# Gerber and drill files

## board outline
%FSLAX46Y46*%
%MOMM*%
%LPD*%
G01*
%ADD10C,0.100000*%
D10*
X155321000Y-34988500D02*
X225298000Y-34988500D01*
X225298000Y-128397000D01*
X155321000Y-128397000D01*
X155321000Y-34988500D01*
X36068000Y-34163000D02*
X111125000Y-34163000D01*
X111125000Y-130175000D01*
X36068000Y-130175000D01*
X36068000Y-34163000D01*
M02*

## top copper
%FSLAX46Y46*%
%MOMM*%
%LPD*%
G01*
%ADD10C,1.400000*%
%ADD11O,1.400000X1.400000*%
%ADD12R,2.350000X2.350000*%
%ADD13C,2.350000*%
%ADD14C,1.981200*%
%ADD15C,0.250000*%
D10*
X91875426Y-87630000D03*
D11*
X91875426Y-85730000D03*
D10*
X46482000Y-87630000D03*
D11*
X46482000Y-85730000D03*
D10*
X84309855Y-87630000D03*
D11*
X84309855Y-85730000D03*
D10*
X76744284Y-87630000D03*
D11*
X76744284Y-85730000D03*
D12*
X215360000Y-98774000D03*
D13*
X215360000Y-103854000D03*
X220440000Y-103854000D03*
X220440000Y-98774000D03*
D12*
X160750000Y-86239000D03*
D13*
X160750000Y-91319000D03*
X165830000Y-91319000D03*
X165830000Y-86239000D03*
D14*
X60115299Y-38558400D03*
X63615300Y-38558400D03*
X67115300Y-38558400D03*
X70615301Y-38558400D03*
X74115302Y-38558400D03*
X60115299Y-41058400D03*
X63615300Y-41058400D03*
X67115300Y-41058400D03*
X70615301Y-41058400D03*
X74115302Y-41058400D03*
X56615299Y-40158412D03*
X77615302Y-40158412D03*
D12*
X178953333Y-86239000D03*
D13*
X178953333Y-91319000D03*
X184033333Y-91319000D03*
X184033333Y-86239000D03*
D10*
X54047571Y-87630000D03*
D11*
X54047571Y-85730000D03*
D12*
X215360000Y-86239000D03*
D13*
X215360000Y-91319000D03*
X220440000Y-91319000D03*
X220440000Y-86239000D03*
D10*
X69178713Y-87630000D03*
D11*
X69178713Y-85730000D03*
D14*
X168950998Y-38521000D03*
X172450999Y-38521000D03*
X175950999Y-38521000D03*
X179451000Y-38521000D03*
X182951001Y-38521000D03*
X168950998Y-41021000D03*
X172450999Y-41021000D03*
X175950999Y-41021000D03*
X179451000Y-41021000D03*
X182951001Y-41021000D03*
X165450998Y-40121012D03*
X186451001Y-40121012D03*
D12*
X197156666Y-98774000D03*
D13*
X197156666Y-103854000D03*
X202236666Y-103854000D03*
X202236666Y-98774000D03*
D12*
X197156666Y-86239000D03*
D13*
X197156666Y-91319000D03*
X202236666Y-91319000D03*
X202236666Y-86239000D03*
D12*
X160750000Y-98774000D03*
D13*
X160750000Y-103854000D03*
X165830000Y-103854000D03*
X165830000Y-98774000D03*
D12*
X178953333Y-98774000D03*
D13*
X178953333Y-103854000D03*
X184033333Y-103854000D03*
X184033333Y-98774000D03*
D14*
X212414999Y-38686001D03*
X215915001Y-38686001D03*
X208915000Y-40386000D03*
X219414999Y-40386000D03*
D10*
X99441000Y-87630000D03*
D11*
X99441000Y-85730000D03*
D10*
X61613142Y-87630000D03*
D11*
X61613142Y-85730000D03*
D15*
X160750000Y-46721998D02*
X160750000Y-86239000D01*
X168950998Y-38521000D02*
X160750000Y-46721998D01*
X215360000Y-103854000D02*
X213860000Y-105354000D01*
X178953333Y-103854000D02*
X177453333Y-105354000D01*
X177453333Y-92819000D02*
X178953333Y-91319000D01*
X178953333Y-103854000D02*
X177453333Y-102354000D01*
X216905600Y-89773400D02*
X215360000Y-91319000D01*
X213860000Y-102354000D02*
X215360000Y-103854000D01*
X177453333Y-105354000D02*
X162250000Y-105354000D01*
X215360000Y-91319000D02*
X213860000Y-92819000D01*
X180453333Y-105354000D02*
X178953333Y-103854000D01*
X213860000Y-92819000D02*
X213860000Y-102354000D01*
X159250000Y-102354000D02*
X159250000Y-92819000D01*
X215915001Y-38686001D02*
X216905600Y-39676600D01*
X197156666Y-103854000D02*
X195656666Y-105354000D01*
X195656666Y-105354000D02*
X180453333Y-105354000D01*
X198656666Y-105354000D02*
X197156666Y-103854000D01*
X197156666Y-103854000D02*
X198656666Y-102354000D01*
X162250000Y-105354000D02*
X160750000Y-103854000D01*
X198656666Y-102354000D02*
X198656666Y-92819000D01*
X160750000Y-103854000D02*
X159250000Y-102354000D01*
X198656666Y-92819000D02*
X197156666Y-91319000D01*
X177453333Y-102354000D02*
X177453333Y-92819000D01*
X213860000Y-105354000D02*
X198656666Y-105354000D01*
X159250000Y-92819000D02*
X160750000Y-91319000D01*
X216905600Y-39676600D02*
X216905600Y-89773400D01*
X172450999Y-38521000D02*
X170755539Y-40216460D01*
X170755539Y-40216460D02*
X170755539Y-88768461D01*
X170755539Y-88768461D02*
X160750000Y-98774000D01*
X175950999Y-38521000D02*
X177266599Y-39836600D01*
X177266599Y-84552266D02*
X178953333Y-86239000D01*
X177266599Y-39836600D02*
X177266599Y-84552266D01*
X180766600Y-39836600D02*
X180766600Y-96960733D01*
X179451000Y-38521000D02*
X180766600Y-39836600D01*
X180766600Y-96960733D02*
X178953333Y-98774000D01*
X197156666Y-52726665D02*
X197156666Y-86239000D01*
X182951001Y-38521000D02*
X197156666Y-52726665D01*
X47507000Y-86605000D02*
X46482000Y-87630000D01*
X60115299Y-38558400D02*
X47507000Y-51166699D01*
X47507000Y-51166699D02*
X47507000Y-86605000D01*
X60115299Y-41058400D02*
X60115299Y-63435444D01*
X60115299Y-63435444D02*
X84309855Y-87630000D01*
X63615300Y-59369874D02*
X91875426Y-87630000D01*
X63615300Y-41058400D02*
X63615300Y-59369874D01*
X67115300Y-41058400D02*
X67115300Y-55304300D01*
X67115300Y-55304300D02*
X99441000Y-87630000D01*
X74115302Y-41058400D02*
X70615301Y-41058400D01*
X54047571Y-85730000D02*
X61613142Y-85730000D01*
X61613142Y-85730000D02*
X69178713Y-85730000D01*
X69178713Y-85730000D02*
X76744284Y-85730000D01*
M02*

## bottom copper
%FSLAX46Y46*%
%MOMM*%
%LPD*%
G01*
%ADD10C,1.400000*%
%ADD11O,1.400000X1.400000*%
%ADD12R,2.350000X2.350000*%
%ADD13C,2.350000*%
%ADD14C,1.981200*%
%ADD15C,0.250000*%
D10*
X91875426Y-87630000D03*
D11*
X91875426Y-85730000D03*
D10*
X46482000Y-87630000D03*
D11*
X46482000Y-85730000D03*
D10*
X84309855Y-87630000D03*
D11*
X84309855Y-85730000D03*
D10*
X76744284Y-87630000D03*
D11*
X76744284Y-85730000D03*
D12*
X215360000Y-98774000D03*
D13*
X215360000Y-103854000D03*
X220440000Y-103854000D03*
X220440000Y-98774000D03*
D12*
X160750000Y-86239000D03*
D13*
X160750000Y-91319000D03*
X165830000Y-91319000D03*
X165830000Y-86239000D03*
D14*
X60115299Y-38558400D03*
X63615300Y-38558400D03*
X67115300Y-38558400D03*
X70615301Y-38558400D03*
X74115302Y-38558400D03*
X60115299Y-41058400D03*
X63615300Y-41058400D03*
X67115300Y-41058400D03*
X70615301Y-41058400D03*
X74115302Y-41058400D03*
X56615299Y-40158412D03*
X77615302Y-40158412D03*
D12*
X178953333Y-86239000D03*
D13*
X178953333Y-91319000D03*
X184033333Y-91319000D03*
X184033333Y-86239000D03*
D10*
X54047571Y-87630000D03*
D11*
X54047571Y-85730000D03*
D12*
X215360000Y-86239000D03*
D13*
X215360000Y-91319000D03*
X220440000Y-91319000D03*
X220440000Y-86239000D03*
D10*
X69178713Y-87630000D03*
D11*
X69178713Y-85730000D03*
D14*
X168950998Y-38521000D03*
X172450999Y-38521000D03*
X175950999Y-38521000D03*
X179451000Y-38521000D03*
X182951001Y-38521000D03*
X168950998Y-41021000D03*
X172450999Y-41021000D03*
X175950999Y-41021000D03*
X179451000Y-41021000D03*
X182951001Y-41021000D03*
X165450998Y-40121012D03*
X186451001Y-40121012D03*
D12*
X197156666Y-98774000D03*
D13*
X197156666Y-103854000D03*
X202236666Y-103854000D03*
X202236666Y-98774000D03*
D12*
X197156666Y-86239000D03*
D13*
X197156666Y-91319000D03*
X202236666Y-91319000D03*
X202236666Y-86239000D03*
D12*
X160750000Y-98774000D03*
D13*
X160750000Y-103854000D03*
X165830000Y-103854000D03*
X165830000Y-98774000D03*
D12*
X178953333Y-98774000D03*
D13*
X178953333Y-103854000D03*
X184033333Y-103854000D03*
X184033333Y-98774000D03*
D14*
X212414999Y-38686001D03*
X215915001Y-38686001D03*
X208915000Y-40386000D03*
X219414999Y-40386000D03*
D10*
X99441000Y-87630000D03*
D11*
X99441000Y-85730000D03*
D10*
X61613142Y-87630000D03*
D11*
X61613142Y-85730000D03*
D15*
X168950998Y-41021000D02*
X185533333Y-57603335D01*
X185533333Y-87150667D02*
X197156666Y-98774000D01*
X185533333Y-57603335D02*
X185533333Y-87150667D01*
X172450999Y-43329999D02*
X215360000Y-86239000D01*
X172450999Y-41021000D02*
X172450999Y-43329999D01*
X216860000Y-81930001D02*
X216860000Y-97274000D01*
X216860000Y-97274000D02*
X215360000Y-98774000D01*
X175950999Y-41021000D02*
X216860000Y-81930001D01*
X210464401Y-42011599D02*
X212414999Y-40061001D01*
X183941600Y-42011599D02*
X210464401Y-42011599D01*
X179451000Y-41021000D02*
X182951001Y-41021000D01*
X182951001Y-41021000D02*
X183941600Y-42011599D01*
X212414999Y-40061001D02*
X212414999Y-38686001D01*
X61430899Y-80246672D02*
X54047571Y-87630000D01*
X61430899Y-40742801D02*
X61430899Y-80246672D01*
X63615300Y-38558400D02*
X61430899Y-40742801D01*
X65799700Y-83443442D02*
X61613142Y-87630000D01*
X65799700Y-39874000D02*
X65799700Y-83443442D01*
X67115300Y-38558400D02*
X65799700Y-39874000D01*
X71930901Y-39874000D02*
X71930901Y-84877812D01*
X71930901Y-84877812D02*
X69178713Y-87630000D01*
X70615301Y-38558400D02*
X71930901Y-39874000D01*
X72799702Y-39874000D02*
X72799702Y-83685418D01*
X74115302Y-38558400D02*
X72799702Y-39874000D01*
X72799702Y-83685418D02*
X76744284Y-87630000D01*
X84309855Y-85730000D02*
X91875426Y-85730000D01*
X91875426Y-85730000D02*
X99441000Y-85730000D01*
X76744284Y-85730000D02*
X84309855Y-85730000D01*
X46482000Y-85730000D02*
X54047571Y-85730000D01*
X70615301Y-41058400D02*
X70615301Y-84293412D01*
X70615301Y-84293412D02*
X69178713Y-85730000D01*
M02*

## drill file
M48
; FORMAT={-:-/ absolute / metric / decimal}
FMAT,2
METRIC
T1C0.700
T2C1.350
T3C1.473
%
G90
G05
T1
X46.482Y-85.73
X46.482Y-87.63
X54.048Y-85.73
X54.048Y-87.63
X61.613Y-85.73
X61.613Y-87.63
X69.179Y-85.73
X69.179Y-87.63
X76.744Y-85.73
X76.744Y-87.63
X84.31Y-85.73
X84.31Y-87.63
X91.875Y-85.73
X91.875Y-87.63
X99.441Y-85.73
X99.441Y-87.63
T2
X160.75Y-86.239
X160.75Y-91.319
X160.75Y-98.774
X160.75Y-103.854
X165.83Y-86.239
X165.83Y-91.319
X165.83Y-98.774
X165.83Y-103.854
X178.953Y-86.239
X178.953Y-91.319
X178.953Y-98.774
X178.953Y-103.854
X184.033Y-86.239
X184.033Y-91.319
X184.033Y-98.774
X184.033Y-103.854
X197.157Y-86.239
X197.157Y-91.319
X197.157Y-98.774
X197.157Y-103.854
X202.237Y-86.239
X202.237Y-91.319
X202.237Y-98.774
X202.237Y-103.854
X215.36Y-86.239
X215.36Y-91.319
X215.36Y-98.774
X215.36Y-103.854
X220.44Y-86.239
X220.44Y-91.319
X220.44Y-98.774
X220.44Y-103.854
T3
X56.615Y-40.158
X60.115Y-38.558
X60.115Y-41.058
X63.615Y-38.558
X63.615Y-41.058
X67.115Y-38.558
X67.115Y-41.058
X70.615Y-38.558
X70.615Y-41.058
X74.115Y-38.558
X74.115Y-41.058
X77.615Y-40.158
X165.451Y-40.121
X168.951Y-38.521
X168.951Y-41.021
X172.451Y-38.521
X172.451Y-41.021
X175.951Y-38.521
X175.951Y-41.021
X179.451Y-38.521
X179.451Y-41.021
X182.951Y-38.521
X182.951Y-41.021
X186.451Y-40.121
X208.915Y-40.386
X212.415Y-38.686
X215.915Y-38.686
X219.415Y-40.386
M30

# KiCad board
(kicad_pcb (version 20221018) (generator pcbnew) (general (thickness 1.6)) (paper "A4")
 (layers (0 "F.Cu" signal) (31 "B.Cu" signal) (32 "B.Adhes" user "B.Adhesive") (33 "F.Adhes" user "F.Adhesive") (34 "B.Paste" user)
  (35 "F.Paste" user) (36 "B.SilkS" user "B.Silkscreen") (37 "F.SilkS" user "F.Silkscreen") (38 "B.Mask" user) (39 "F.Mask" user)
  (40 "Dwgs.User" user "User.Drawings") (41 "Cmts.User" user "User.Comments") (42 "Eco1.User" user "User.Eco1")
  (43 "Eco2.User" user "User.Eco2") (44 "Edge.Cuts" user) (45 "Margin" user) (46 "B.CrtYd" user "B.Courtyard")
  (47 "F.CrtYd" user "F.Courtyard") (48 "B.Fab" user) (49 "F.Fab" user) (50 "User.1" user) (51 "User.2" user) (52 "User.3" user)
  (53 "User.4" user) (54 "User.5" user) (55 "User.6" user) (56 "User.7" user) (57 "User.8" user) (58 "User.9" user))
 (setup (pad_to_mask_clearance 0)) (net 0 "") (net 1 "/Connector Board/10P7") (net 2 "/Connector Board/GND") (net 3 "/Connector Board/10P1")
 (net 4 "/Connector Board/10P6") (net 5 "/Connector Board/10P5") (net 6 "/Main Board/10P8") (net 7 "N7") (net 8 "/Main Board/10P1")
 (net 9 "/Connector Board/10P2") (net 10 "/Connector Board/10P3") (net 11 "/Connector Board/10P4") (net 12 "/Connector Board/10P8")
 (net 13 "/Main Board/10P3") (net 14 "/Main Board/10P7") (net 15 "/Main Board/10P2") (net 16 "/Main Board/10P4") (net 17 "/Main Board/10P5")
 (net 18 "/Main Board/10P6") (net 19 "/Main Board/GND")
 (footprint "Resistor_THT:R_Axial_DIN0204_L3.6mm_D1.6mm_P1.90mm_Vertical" (layer "F.Cu") (at 91.875426 87.63 90)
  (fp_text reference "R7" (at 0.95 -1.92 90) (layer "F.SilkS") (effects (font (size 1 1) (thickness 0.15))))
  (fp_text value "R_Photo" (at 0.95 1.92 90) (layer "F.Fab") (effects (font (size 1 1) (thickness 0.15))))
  (pad "1" thru_hole circle (at 0 0 90) (size 1.4 1.4) (drill 0.7) (layers "*.Cu" "*.Mask") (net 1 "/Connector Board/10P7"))
  (pad "2" thru_hole oval (at 1.9 0 90) (size 1.4 1.4) (drill 0.7) (layers "*.Cu" "*.Mask") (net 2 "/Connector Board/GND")))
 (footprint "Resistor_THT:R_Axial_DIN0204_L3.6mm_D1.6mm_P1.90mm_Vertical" (layer "F.Cu") (at 46.482 87.63 90)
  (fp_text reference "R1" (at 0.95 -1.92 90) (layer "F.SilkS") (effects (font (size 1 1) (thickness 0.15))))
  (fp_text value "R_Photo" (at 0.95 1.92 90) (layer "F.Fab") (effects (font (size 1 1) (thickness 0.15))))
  (pad "1" thru_hole circle (at 0 0 90) (size 1.4 1.4) (drill 0.7) (layers "*.Cu" "*.Mask") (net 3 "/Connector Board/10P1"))
  (pad "2" thru_hole oval (at 1.9 0 90) (size 1.4 1.4) (drill 0.7) (layers "*.Cu" "*.Mask") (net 2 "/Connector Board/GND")))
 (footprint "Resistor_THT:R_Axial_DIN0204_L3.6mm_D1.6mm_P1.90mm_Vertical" (layer "F.Cu") (at 84.309855 87.63 90)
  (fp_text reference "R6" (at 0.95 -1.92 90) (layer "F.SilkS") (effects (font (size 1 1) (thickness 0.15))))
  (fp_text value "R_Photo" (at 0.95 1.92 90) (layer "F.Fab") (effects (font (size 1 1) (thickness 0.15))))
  (pad "1" thru_hole circle (at 0 0 90) (size 1.4 1.4) (drill 0.7) (layers "*.Cu" "*.Mask") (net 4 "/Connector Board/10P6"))
  (pad "2" thru_hole oval (at 1.9 0 90) (size 1.4 1.4) (drill 0.7) (layers "*.Cu" "*.Mask") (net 2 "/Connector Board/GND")))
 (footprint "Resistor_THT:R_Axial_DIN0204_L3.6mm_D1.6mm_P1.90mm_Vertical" (layer "F.Cu") (at 76.744284 87.63 90)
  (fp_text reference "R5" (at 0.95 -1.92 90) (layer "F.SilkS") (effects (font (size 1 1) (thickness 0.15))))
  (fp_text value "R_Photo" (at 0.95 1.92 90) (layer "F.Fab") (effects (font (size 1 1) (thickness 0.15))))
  (pad "1" thru_hole circle (at 0 0 90) (size 1.4 1.4) (drill 0.7) (layers "*.Cu" "*.Mask") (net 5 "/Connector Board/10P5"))
  (pad "2" thru_hole oval (at 1.9 0 90) (size 1.4 1.4) (drill 0.7) (layers "*.Cu" "*.Mask") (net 2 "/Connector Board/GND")))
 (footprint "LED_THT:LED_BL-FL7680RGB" (layer "F.Cu") (at 215.36 98.774)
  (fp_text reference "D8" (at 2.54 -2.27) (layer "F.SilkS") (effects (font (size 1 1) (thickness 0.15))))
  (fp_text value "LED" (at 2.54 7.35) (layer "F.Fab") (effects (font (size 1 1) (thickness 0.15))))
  (pad "1" thru_hole rect (at 0 0) (size 2.35 2.35) (drill 1.35) (layers "*.Cu" "*.Mask") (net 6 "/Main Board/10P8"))
  (pad "2" thru_hole circle (at 0 5.08) (size 2.35 2.35) (drill 1.35) (layers "*.Cu" "*.Mask") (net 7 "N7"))
  (pad "3" thru_hole circle (at 5.08 5.08) (size 2.35 2.35) (drill 1.35) (layers "*.Cu" "*.Mask"))
  (pad "4" thru_hole circle (at 5.08 0) (size 2.35 2.35) (drill 1.35) (layers "*.Cu" "*.Mask")))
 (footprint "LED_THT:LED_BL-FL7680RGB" (layer "F.Cu") (at 160.75 86.239)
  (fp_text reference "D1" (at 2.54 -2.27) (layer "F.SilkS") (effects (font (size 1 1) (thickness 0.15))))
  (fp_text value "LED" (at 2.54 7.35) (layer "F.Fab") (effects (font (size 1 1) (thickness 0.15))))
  (pad "1" thru_hole rect (at 0 0) (size 2.35 2.35) (drill 1.35) (layers "*.Cu" "*.Mask") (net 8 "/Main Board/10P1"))
  (pad "2" thru_hole circle (at 0 5.08) (size 2.35 2.35) (drill 1.35) (layers "*.Cu" "*.Mask") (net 7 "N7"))
  (pad "3" thru_hole circle (at 5.08 5.08) (size 2.35 2.35) (drill 1.35) (layers "*.Cu" "*.Mask"))
  (pad "4" thru_hole circle (at 5.08 0) (size 2.35 2.35) (drill 1.35) (layers "*.Cu" "*.Mask")))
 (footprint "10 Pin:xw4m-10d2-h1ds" (layer "F.Cu") (at 60.115299 38.5584)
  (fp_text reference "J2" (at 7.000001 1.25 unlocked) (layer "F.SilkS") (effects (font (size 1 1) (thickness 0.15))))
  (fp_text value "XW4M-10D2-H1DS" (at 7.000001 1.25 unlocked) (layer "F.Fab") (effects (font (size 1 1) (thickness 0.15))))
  (pad "1" thru_hole circle (at 0 0) (size 1.9812 1.9812) (drill 1.4732) (layers "*.Cu" "*.Mask") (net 3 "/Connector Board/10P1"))
  (pad "2" thru_hole circle (at 3.500001 0) (size 1.9812 1.9812) (drill 1.4732) (layers "*.Cu" "*.Mask") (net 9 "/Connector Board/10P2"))
  (pad "3" thru_hole circle (at 7.000001 0) (size 1.9812 1.9812) (drill 1.4732) (layers "*.Cu" "*.Mask") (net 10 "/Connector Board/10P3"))
  (pad "4" thru_hole circle (at 10.500002 0) (size 1.9812 1.9812) (drill 1.4732) (layers "*.Cu" "*.Mask") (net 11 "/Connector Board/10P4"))
  (pad "5" thru_hole circle (at 14.000003 0) (size 1.9812 1.9812) (drill 1.4732) (layers "*.Cu" "*.Mask") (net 5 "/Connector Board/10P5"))
  (pad "6" thru_hole circle (at 0 2.5) (size 1.9812 1.9812) (drill 1.4732) (layers "*.Cu" "*.Mask") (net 4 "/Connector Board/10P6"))
  (pad "7" thru_hole circle (at 3.500001 2.5) (size 1.9812 1.9812) (drill 1.4732) (layers "*.Cu" "*.Mask") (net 1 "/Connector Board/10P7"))
  (pad "8" thru_hole circle (at 7.000001 2.5) (size 1.9812 1.9812) (drill 1.4732) (layers "*.Cu" "*.Mask") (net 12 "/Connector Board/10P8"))
  (pad "9" thru_hole circle (at 10.500002 2.5) (size 1.9812 1.9812) (drill 1.4732) (layers "*.Cu" "*.Mask") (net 2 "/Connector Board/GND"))
  (pad "10" thru_hole circle (at 14.000003 2.5) (size 1.9812 1.9812) (drill 1.4732) (layers "*.Cu" "*.Mask") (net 2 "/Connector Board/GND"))
  (pad "11" thru_hole circle (at -3.5 1.600012) (size 1.9812 1.9812) (drill 1.4732) (layers "*.Cu" "*.Mask"))
  (pad "12" thru_hole circle (at 17.500003 1.600012) (size 1.9812 1.9812) (drill 1.4732) (layers "*.Cu" "*.Mask")))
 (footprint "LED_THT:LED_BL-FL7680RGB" (layer "F.Cu") (at 178.953333 86.239)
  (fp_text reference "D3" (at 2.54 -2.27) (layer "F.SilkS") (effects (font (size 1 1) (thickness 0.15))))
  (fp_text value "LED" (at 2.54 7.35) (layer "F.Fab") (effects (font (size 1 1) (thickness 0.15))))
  (pad "1" thru_hole rect (at 0 0) (size 2.35 2.35) (drill 1.35) (layers "*.Cu" "*.Mask") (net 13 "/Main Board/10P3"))
  (pad "2" thru_hole circle (at 0 5.08) (size 2.35 2.35) (drill 1.35) (layers "*.Cu" "*.Mask") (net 7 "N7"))
  (pad "3" thru_hole circle (at 5.08 5.08) (size 2.35 2.35) (drill 1.35) (layers "*.Cu" "*.Mask"))
  (pad "4" thru_hole circle (at 5.08 0) (size 2.35 2.35) (drill 1.35) (layers "*.Cu" "*.Mask")))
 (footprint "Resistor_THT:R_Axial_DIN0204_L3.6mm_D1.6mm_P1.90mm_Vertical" (layer "F.Cu") (at 54.047571 87.63 90)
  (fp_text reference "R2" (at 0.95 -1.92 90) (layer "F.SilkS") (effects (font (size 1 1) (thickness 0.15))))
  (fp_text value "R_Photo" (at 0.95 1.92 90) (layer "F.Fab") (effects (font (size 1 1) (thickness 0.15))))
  (pad "1" thru_hole circle (at 0 0 90) (size 1.4 1.4) (drill 0.7) (layers "*.Cu" "*.Mask") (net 9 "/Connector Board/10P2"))
  (pad "2" thru_hole oval (at 1.9 0 90) (size 1.4 1.4) (drill 0.7) (layers "*.Cu" "*.Mask") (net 2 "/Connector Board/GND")))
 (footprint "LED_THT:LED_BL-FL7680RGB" (layer "F.Cu") (at 215.36 86.239)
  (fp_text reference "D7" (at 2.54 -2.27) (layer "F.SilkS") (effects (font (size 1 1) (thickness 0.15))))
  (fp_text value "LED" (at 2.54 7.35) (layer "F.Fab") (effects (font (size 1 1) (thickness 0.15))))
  (pad "1" thru_hole rect (at 0 0) (size 2.35 2.35) (drill 1.35) (layers "*.Cu" "*.Mask") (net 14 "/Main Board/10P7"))
  (pad "2" thru_hole circle (at 0 5.08) (size 2.35 2.35) (drill 1.35) (layers "*.Cu" "*.Mask") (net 7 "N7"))
  (pad "3" thru_hole circle (at 5.08 5.08) (size 2.35 2.35) (drill 1.35) (layers "*.Cu" "*.Mask"))
  (pad "4" thru_hole circle (at 5.08 0) (size 2.35 2.35) (drill 1.35) (layers "*.Cu" "*.Mask")))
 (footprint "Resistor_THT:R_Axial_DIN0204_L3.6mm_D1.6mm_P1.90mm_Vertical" (layer "F.Cu") (at 69.178713 87.63 90)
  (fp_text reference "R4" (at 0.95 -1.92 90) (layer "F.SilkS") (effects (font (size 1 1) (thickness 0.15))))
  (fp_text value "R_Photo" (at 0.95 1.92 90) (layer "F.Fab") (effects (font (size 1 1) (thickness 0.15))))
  (pad "1" thru_hole circle (at 0 0 90) (size 1.4 1.4) (drill 0.7) (layers "*.Cu" "*.Mask") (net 11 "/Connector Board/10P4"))
  (pad "2" thru_hole oval (at 1.9 0 90) (size 1.4 1.4) (drill 0.7) (layers "*.Cu" "*.Mask") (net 2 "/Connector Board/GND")))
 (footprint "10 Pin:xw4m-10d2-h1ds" (layer "F.Cu") (at 168.950998 38.521)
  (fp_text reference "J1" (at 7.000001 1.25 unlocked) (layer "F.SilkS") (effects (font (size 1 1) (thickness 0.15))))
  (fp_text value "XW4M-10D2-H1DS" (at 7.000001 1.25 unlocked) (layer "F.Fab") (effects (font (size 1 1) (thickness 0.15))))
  (pad "1" thru_hole circle (at 0 0) (size 1.9812 1.9812) (drill 1.4732) (layers "*.Cu" "*.Mask") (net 8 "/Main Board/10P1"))
  (pad "2" thru_hole circle (at 3.500001 0) (size 1.9812 1.9812) (drill 1.4732) (layers "*.Cu" "*.Mask") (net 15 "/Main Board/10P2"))
  (pad "3" thru_hole circle (at 7.000001 0) (size 1.9812 1.9812) (drill 1.4732) (layers "*.Cu" "*.Mask") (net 13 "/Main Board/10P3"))
  (pad "4" thru_hole circle (at 10.500002 0) (size 1.9812 1.9812) (drill 1.4732) (layers "*.Cu" "*.Mask") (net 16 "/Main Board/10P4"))
  (pad "5" thru_hole circle (at 14.000003 0) (size 1.9812 1.9812) (drill 1.4732) (layers "*.Cu" "*.Mask") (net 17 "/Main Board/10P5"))
  (pad "6" thru_hole circle (at 0 2.5) (size 1.9812 1.9812) (drill 1.4732) (layers "*.Cu" "*.Mask") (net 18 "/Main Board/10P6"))
  (pad "7" thru_hole circle (at 3.500001 2.5) (size 1.9812 1.9812) (drill 1.4732) (layers "*.Cu" "*.Mask") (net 14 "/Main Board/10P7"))
  (pad "8" thru_hole circle (at 7.000001 2.5) (size 1.9812 1.9812) (drill 1.4732) (layers "*.Cu" "*.Mask") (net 6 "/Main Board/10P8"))
  (pad "9" thru_hole circle (at 10.500002 2.5) (size 1.9812 1.9812) (drill 1.4732) (layers "*.Cu" "*.Mask") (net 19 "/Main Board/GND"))
  (pad "10" thru_hole circle (at 14.000003 2.5) (size 1.9812 1.9812) (drill 1.4732) (layers "*.Cu" "*.Mask") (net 19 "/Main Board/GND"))
  (pad "11" thru_hole circle (at -3.5 1.600012) (size 1.9812 1.9812) (drill 1.4732) (layers "*.Cu" "*.Mask"))
  (pad "12" thru_hole circle (at 17.500003 1.600012) (size 1.9812 1.9812) (drill 1.4732) (layers "*.Cu" "*.Mask")))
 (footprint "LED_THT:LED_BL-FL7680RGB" (layer "F.Cu") (at 197.156666 98.774)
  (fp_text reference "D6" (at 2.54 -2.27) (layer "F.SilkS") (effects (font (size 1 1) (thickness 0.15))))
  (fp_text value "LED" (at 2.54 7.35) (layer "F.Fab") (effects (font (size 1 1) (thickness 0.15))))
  (pad "1" thru_hole rect (at 0 0) (size 2.35 2.35) (drill 1.35) (layers "*.Cu" "*.Mask") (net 18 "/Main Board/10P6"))
  (pad "2" thru_hole circle (at 0 5.08) (size 2.35 2.35) (drill 1.35) (layers "*.Cu" "*.Mask") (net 7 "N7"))
  (pad "3" thru_hole circle (at 5.08 5.08) (size 2.35 2.35) (drill 1.35) (layers "*.Cu" "*.Mask"))
  (pad "4" thru_hole circle (at 5.08 0) (size 2.35 2.35) (drill 1.35) (layers "*.Cu" "*.Mask")))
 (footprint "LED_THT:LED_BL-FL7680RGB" (layer "F.Cu") (at 197.156666 86.239)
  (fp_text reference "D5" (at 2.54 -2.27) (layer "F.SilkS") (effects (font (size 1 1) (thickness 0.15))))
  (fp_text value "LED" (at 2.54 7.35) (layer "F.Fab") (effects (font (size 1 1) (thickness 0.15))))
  (pad "1" thru_hole rect (at 0 0) (size 2.35 2.35) (drill 1.35) (layers "*.Cu" "*.Mask") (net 17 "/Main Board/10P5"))
  (pad "2" thru_hole circle (at 0 5.08) (size 2.35 2.35) (drill 1.35) (layers "*.Cu" "*.Mask") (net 7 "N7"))
  (pad "3" thru_hole circle (at 5.08 5.08) (size 2.35 2.35) (drill 1.35) (layers "*.Cu" "*.Mask"))
  (pad "4" thru_hole circle (at 5.08 0) (size 2.35 2.35) (drill 1.35) (layers "*.Cu" "*.Mask")))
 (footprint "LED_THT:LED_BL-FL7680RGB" (layer "F.Cu") (at 160.75 98.774)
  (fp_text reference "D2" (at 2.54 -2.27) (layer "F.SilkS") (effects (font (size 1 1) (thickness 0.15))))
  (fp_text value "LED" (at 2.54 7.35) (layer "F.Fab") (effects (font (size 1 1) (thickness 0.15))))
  (pad "1" thru_hole rect (at 0 0) (size 2.35 2.35) (drill 1.35) (layers "*.Cu" "*.Mask") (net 15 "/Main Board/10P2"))
  (pad "2" thru_hole circle (at 0 5.08) (size 2.35 2.35) (drill 1.35) (layers "*.Cu" "*.Mask") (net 7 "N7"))
  (pad "3" thru_hole circle (at 5.08 5.08) (size 2.35 2.35) (drill 1.35) (layers "*.Cu" "*.Mask"))
  (pad "4" thru_hole circle (at 5.08 0) (size 2.35 2.35) (drill 1.35) (layers "*.Cu" "*.Mask")))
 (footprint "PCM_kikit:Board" (layer "F.Cu") (at 36.322 34.163)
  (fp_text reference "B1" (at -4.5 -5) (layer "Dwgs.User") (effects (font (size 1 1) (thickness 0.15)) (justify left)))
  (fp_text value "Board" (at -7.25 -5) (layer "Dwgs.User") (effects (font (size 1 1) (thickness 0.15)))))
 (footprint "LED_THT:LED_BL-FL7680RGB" (layer "F.Cu") (at 178.953333 98.774)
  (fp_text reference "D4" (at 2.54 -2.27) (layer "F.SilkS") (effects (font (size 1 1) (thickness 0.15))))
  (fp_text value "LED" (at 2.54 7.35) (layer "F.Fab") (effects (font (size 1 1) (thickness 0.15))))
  (pad "1" thru_hole rect (at 0 0) (size 2.35 2.35) (drill 1.35) (layers "*.Cu" "*.Mask") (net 16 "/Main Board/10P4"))
  (pad "2" thru_hole circle (at 0 5.08) (size 2.35 2.35) (drill 1.35) (layers "*.Cu" "*.Mask") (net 7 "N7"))
  (pad "3" thru_hole circle (at 5.08 5.08) (size 2.35 2.35) (drill 1.35) (layers "*.Cu" "*.Mask"))
  (pad "4" thru_hole circle (at 5.08 0) (size 2.35 2.35) (drill 1.35) (layers "*.Cu" "*.Mask")))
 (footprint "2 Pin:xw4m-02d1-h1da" (layer "F.Cu") (at 212.414999 38.686001)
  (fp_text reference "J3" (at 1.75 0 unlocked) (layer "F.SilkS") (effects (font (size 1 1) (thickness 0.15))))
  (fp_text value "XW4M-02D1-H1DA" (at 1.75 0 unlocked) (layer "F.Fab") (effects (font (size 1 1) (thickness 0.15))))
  (pad "1" thru_hole circle (at 0 0) (size 1.9812 1.9812) (drill 1.4732) (layers "*.Cu" "*.Mask") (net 19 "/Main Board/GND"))
  (pad "2" thru_hole circle (at 3.500002 0) (size 1.9812 1.9812) (drill 1.4732) (layers "*.Cu" "*.Mask") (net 7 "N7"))
  (pad "3" thru_hole circle (at -3.499999 1.699999) (size 1.9812 1.9812) (drill 1.4732) (layers "*.Cu" "*.Mask"))
  (pad "4" thru_hole circle (at 7 1.699999) (size 1.9812 1.9812) (drill 1.4732) (layers "*.Cu" "*.Mask")))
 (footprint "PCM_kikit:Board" (layer "F.Cu") (at 158.496 34.8615)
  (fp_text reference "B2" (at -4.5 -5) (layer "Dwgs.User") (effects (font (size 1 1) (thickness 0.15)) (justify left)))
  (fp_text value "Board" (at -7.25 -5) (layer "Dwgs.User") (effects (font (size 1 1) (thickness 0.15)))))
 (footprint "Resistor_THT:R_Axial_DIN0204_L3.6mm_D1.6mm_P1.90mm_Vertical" (layer "F.Cu") (at 99.441 87.63 90)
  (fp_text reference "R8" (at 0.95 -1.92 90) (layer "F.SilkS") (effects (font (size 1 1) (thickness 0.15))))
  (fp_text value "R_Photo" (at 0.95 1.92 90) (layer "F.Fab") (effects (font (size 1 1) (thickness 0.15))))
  (pad "1" thru_hole circle (at 0 0 90) (size 1.4 1.4) (drill 0.7) (layers "*.Cu" "*.Mask") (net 12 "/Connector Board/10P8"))
  (pad "2" thru_hole oval (at 1.9 0 90) (size 1.4 1.4) (drill 0.7) (layers "*.Cu" "*.Mask") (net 2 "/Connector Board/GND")))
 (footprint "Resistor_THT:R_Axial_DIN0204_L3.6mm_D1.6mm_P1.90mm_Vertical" (layer "F.Cu") (at 61.613142 87.63 90)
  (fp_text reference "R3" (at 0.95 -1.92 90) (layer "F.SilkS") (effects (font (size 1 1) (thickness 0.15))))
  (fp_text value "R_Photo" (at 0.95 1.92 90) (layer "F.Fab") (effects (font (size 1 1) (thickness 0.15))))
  (pad "1" thru_hole circle (at 0 0 90) (size 1.4 1.4) (drill 0.7) (layers "*.Cu" "*.Mask") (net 10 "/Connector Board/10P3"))
  (pad "2" thru_hole oval (at 1.9 0 90) (size 1.4 1.4) (drill 0.7) (layers "*.Cu" "*.Mask") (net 2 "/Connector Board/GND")))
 (gr_rect (start 155.321 34.9885) (end 225.298 128.397) (stroke (width 0.1) (type default)) (fill none) (layer "Edge.Cuts"))
 (gr_rect (start 36.068 34.163) (end 111.125 130.175) (stroke (width 0.1) (type default)) (fill none) (layer "Edge.Cuts"))
 (segment (start 160.75 46.721998) (end 160.75 86.239) (width 0.25) (layer "F.Cu") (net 8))
 (segment (start 168.950998 38.521) (end 160.75 46.721998) (width 0.25) (layer "F.Cu") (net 8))
 (segment (start 215.36 103.854) (end 213.86 105.354) (width 0.25) (layer "F.Cu") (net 7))
 (segment (start 178.953333 103.854) (end 177.453333 105.354) (width 0.25) (layer "F.Cu") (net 7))
 (segment (start 177.453333 92.819) (end 178.953333 91.319) (width 0.25) (layer "F.Cu") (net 7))
 (segment (start 178.953333 103.854) (end 177.453333 102.354) (width 0.25) (layer "F.Cu") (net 7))
 (segment (start 216.9056 89.7734) (end 215.36 91.319) (width 0.25) (layer "F.Cu") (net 7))
 (segment (start 213.86 102.354) (end 215.36 103.854) (width 0.25) (layer "F.Cu") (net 7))
 (segment (start 177.453333 105.354) (end 162.25 105.354) (width 0.25) (layer "F.Cu") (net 7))
 (segment (start 215.36 91.319) (end 213.86 92.819) (width 0.25) (layer "F.Cu") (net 7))
 (segment (start 180.453333 105.354) (end 178.953333 103.854) (width 0.25) (layer "F.Cu") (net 7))
 (segment (start 213.86 92.819) (end 213.86 102.354) (width 0.25) (layer "F.Cu") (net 7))
 (segment (start 159.25 102.354) (end 159.25 92.819) (width 0.25) (layer "F.Cu") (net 7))
 (segment (start 215.915001 38.686001) (end 216.9056 39.6766) (width 0.25) (layer "F.Cu") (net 7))
 (segment (start 197.156666 103.854) (end 195.656666 105.354) (width 0.25) (layer "F.Cu") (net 7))
 (segment (start 195.656666 105.354) (end 180.453333 105.354) (width 0.25) (layer "F.Cu") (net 7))
 (segment (start 198.656666 105.354) (end 197.156666 103.854) (width 0.25) (layer "F.Cu") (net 7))
 (segment (start 197.156666 103.854) (end 198.656666 102.354) (width 0.25) (layer "F.Cu") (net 7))
 (segment (start 162.25 105.354) (end 160.75 103.854) (width 0.25) (layer "F.Cu") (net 7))
 (segment (start 198.656666 102.354) (end 198.656666 92.819) (width 0.25) (layer "F.Cu") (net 7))
 (segment (start 160.75 103.854) (end 159.25 102.354) (width 0.25) (layer "F.Cu") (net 7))
 (segment (start 198.656666 92.819) (end 197.156666 91.319) (width 0.25) (layer "F.Cu") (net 7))
 (segment (start 177.453333 102.354) (end 177.453333 92.819) (width 0.25) (layer "F.Cu") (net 7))
 (segment (start 213.86 105.354) (end 198.656666 105.354) (width 0.25) (layer "F.Cu") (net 7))
 (segment (start 159.25 92.819) (end 160.75 91.319) (width 0.25) (layer "F.Cu") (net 7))
 (segment (start 216.9056 39.6766) (end 216.9056 89.7734) (width 0.25) (layer "F.Cu") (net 7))
 (segment (start 172.450999 38.521) (end 170.755539 40.21646) (width 0.25) (layer "F.Cu") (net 15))
 (segment (start 170.755539 40.21646) (end 170.755539 88.768461) (width 0.25) (layer "F.Cu") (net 15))
 (segment (start 170.755539 88.768461) (end 160.75 98.774) (width 0.25) (layer "F.Cu") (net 15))
 (segment (start 175.950999 38.521) (end 177.266599 39.8366) (width 0.25) (layer "F.Cu") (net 13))
 (segment (start 177.266599 84.552266) (end 178.953333 86.239) (width 0.25) (layer "F.Cu") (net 13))
 (segment (start 177.266599 39.8366) (end 177.266599 84.552266) (width 0.25) (layer "F.Cu") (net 13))
 (segment (start 180.7666 39.8366) (end 180.7666 96.960733) (width 0.25) (layer "F.Cu") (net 16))
 (segment (start 179.451 38.521) (end 180.7666 39.8366) (width 0.25) (layer "F.Cu") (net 16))
 (segment (start 180.7666 96.960733) (end 178.953333 98.774) (width 0.25) (layer "F.Cu") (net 16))
 (segment (start 197.156666 52.726665) (end 197.156666 86.239) (width 0.25) (layer "F.Cu") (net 17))
 (segment (start 182.951001 38.521) (end 197.156666 52.726665) (width 0.25) (layer "F.Cu") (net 17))
 (segment (start 168.950998 41.021) (end 185.533333 57.603335) (width 0.25) (layer "B.Cu") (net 18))
 (segment (start 185.533333 87.150667) (end 197.156666 98.774) (width 0.25) (layer "B.Cu") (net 18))
 (segment (start 185.533333 57.603335) (end 185.533333 87.150667) (width 0.25) (layer "B.Cu") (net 18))
 (segment (start 172.450999 43.329999) (end 215.36 86.239) (width 0.25) (layer "B.Cu") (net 14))
 (segment (start 172.450999 41.021) (end 172.450999 43.329999) (width 0.25) (layer "B.Cu") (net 14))
 (segment (start 216.86 81.930001) (end 216.86 97.274) (width 0.25) (layer "B.Cu") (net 6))
 (segment (start 216.86 97.274) (end 215.36 98.774) (width 0.25) (layer "B.Cu") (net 6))
 (segment (start 175.950999 41.021) (end 216.86 81.930001) (width 0.25) (layer "B.Cu") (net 6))
 (segment (start 210.464401 42.011599) (end 212.414999 40.061001) (width 0.25) (layer "B.Cu") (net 19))
 (segment (start 183.9416 42.011599) (end 210.464401 42.011599) (width 0.25) (layer "B.Cu") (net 19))
 (segment (start 179.451 41.021) (end 182.951001 41.021) (width 0.25) (layer "B.Cu") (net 19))
 (segment (start 182.951001 41.021) (end 183.9416 42.011599) (width 0.25) (layer "B.Cu") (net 19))
 (segment (start 212.414999 40.061001) (end 212.414999 38.686001) (width 0.25) (layer "B.Cu") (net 19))
 (segment (start 47.507 86.605) (end 46.482 87.63) (width 0.25) (layer "F.Cu") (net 3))
 (segment (start 60.115299 38.5584) (end 47.507 51.166699) (width 0.25) (layer "F.Cu") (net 3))
 (segment (start 47.507 51.166699) (end 47.507 86.605) (width 0.25) (layer "F.Cu") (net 3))
 (segment (start 61.430899 80.246672) (end 54.047571 87.63) (width 0.25) (layer "B.Cu") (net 9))
 (segment (start 61.430899 40.742801) (end 61.430899 80.246672) (width 0.25) (layer "B.Cu") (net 9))
 (segment (start 63.6153 38.5584) (end 61.430899 40.742801) (width 0.25) (layer "B.Cu") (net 9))
 (segment (start 65.7997 83.443442) (end 61.613142 87.63) (width 0.25) (layer "B.Cu") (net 10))
 (segment (start 65.7997 39.874) (end 65.7997 83.443442) (width 0.25) (layer "B.Cu") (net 10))
 (segment (start 67.1153 38.5584) (end 65.7997 39.874) (width 0.25) (layer "B.Cu") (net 10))
 (segment (start 71.930901 39.874) (end 71.930901 84.877812) (width 0.25) (layer "B.Cu") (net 11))
 (segment (start 71.930901 84.877812) (end 69.178713 87.63) (width 0.25) (layer "B.Cu") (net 11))
 (segment (start 70.615301 38.5584) (end 71.930901 39.874) (width 0.25) (layer "B.Cu") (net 11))
 (segment (start 72.799702 39.874) (end 72.799702 83.685418) (width 0.25) (layer "B.Cu") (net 5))
 (segment (start 74.115302 38.5584) (end 72.799702 39.874) (width 0.25) (layer "B.Cu") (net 5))
 (segment (start 72.799702 83.685418) (end 76.744284 87.63) (width 0.25) (layer "B.Cu") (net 5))
 (segment (start 60.115299 41.0584) (end 60.115299 63.435444) (width 0.25) (layer "F.Cu") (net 4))
 (segment (start 60.115299 63.435444) (end 84.309855 87.63) (width 0.25) (layer "F.Cu") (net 4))
 (segment (start 63.6153 59.369874) (end 91.875426 87.63) (width 0.25) (layer "F.Cu") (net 1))
 (segment (start 63.6153 41.0584) (end 63.6153 59.369874) (width 0.25) (layer "F.Cu") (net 1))
 (segment (start 67.1153 41.0584) (end 67.1153 55.3043) (width 0.25) (layer "F.Cu") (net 12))
 (segment (start 67.1153 55.3043) (end 99.441 87.63) (width 0.25) (layer "F.Cu") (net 12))
 (segment (start 74.115302 41.0584) (end 70.615301 41.0584) (width 0.25) (layer "F.Cu") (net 2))
 (segment (start 54.047571 85.73) (end 61.613142 85.73) (width 0.25) (layer "F.Cu") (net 2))
 (segment (start 61.613142 85.73) (end 69.178713 85.73) (width 0.25) (layer "F.Cu") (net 2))
 (segment (start 69.178713 85.73) (end 76.744284 85.73) (width 0.25) (layer "F.Cu") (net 2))
 (segment (start 84.309855 85.73) (end 91.875426 85.73) (width 0.25) (layer "B.Cu") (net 2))
 (segment (start 91.875426 85.73) (end 99.441 85.73) (width 0.25) (layer "B.Cu") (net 2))
 (segment (start 76.744284 85.73) (end 84.309855 85.73) (width 0.25) (layer "B.Cu") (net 2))
 (segment (start 46.482 85.73) (end 54.047571 85.73) (width 0.25) (layer "B.Cu") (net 2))
 (segment (start 70.615301 41.0584) (end 70.615301 84.293412) (width 0.25) (layer "B.Cu") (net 2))
 (segment (start 70.615301 84.293412) (end 69.178713 85.73) (width 0.25) (layer "B.Cu") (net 2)))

